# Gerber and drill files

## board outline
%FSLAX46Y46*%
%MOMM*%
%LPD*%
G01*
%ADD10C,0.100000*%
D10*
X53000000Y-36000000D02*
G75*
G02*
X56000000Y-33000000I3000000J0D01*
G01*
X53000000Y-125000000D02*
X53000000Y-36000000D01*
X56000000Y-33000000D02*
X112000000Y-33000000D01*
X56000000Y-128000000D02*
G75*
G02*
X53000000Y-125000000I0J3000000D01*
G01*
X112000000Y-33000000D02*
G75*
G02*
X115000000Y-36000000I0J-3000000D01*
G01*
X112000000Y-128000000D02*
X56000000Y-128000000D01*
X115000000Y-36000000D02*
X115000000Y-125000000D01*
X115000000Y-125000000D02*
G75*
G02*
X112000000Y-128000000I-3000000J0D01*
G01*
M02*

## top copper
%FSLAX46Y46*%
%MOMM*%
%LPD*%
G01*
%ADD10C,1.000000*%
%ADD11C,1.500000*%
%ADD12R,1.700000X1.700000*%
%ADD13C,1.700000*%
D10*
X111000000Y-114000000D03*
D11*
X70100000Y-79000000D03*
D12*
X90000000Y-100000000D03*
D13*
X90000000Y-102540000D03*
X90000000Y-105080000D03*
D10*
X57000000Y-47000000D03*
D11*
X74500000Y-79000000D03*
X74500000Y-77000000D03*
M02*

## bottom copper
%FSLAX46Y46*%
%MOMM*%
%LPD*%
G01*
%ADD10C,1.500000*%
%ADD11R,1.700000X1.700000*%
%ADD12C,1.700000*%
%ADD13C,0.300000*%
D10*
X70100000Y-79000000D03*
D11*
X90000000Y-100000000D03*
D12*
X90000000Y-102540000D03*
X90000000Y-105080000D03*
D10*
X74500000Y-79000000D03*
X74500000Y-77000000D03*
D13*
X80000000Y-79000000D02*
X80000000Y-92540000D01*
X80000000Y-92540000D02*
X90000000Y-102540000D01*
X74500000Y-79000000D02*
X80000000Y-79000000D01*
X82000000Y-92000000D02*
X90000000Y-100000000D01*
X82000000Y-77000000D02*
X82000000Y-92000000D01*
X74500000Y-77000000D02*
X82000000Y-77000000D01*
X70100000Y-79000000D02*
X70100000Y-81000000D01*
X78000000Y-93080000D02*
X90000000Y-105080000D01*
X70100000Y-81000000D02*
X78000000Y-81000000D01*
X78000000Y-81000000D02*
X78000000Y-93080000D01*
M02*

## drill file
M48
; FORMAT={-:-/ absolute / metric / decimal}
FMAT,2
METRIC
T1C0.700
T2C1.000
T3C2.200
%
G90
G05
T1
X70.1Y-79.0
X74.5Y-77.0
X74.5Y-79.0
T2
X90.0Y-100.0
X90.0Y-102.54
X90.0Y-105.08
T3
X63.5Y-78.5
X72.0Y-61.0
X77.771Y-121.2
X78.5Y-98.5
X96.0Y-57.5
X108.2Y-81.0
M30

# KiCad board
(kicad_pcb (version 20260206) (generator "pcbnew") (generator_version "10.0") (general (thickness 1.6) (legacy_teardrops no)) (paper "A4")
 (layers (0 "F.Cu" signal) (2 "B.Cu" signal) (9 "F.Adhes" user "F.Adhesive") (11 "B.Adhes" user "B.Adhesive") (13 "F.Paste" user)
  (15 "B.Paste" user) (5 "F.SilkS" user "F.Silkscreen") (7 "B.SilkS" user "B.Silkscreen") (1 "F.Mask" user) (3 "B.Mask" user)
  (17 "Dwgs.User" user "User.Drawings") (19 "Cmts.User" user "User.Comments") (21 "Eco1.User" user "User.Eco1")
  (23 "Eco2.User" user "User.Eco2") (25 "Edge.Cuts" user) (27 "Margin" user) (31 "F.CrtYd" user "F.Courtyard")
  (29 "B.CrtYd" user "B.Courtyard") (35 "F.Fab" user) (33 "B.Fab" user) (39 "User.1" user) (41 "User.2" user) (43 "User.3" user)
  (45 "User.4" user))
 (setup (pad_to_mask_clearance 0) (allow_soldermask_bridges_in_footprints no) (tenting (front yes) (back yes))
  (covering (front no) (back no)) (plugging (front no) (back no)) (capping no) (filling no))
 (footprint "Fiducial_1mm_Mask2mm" (layer "F.Cu") (at 111 114)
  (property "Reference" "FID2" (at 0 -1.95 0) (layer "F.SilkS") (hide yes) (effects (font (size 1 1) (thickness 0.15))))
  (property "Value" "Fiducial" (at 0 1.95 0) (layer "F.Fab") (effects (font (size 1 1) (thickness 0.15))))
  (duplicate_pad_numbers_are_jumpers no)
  (pad "" smd circle (at 0 0) (size 1 1) (layers "F.Cu" "F.Mask") (solder_mask_margin 0.5) (clearance 0.6)))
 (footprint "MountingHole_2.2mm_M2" (layer "F.Cu") (at 77.771 121.2)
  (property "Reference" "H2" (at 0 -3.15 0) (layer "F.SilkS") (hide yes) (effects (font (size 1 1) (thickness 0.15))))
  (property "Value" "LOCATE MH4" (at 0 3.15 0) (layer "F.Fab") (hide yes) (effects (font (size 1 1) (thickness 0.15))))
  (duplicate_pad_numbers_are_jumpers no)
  (pad "" np_thru_hole circle (at 0 0) (size 2.2 2.2) (drill 2.2) (layers "*.Cu" "*.Mask")))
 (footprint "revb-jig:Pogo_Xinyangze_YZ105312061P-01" (layer "F.Cu") (at 70.1 79)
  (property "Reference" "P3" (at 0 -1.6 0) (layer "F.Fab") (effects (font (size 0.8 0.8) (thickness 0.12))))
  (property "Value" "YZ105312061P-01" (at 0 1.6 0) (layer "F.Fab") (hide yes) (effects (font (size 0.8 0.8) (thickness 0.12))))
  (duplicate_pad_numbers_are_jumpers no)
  (pad "1" thru_hole circle (at 0 0) (size 1.5 1.5) (drill 0.7) (layers "*.Cu" "*.Mask" "F.Paste") (remove_unused_layers no) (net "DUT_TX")))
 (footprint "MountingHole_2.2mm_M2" (layer "F.Cu") (at 108.2 81)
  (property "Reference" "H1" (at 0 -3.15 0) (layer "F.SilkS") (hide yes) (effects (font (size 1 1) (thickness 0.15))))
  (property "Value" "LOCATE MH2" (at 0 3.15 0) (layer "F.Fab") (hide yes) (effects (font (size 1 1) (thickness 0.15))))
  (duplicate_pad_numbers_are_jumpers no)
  (pad "" np_thru_hole circle (at 0 0) (size 2.2 2.2) (drill 2.2) (layers "*.Cu" "*.Mask")))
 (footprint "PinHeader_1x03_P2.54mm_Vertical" (layer "F.Cu") (at 90 100)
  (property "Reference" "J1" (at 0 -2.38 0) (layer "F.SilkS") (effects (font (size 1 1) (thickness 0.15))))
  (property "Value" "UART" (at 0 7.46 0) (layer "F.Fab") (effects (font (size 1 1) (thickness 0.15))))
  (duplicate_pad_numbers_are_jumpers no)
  (pad "1" thru_hole rect (at 0 0) (size 1.7 1.7) (drill 1) (layers "*.Cu" "*.Mask") (remove_unused_layers no) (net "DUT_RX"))
  (pad "2" thru_hole circle (at 0 2.54) (size 1.7 1.7) (drill 1) (layers "*.Cu" "*.Mask") (remove_unused_layers no) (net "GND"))
  (pad "3" thru_hole circle (at 0 5.08) (size 1.7 1.7) (drill 1) (layers "*.Cu" "*.Mask") (remove_unused_layers no) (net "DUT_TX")))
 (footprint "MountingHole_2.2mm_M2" (layer "F.Cu") (at 96 57.5)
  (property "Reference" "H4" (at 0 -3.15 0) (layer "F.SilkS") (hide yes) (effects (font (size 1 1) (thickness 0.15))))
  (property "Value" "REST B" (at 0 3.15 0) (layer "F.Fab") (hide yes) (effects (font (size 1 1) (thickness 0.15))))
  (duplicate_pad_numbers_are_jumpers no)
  (pad "" np_thru_hole circle (at 0 0) (size 2.2 2.2) (drill 2.2) (layers "*.Cu" "*.Mask")))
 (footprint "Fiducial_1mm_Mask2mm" (layer "F.Cu") (at 57 47)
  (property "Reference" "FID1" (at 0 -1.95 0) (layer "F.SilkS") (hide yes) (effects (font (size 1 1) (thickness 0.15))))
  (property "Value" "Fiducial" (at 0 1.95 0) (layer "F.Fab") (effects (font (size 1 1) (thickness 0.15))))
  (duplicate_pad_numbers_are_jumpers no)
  (pad "" smd circle (at 0 0) (size 1 1) (layers "F.Cu" "F.Mask") (solder_mask_margin 0.5) (clearance 0.6)))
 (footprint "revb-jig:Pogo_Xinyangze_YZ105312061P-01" (layer "F.Cu") (at 74.5 79)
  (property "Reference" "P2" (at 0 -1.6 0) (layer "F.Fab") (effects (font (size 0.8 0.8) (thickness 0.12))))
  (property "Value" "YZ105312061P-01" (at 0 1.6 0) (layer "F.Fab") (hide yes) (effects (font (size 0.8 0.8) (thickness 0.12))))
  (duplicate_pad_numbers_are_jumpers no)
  (pad "1" thru_hole circle (at 0 0) (size 1.5 1.5) (drill 0.7) (layers "*.Cu" "*.Mask" "F.Paste") (remove_unused_layers no) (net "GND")))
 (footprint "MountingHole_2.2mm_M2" (layer "F.Cu") (at 78.5 98.5)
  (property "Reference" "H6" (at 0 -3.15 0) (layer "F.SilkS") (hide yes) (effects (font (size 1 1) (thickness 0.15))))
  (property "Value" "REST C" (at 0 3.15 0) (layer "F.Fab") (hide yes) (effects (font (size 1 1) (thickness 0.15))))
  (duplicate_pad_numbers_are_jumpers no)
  (pad "" np_thru_hole circle (at 0 0) (size 2.2 2.2) (drill 2.2) (layers "*.Cu" "*.Mask")))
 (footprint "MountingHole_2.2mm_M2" (layer "F.Cu") (at 72 61)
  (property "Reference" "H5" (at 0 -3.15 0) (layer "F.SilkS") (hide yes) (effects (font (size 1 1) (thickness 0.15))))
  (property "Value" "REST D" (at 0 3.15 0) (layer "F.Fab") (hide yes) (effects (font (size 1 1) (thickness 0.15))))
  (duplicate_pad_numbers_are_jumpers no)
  (pad "" np_thru_hole circle (at 0 0) (size 2.2 2.2) (drill 2.2) (layers "*.Cu" "*.Mask")))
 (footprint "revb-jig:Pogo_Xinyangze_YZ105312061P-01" (layer "F.Cu") (at 74.5 77)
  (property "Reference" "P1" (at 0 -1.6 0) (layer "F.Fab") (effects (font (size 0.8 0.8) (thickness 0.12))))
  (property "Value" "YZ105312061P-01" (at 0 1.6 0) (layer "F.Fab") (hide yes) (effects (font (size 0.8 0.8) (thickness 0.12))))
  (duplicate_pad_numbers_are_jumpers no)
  (pad "1" thru_hole circle (at 0 0) (size 1.5 1.5) (drill 0.7) (layers "*.Cu" "*.Mask" "F.Paste") (remove_unused_layers no) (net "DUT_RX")))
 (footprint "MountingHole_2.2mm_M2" (layer "F.Cu") (at 63.5 78.5)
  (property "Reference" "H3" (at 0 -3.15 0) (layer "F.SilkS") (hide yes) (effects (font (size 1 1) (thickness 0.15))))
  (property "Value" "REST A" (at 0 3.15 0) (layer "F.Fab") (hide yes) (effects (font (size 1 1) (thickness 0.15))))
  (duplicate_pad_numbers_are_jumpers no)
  (pad "" np_thru_hole circle (at 0 0) (size 2.2 2.2) (drill 2.2) (layers "*.Cu" "*.Mask")))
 (gr_arc (start 53 36) (mid 53.878679 33.878679) (end 56 33) (stroke (width 0.1) (type default)) (layer "Edge.Cuts"))
 (gr_line (start 53 125) (end 53 36) (stroke (width 0.1) (type default)) (layer "Edge.Cuts"))
 (gr_line (start 56 33) (end 112 33) (stroke (width 0.1) (type default)) (layer "Edge.Cuts"))
 (gr_arc (start 56 128) (mid 53.878679 127.12132) (end 53 125) (stroke (width 0.1) (type default)) (layer "Edge.Cuts"))
 (gr_arc (start 112 33) (mid 114.12132 33.878679) (end 115 36) (stroke (width 0.1) (type default)) (layer "Edge.Cuts"))
 (gr_line (start 112 128) (end 56 128) (stroke (width 0.1) (type default)) (layer "Edge.Cuts"))
 (gr_line (start 115 36) (end 115 125) (stroke (width 0.1) (type default)) (layer "Edge.Cuts"))
 (gr_arc (start 115 125) (mid 114.12132 127.12132) (end 112 128) (stroke (width 0.1) (type default)) (layer "Edge.Cuts"))
 (segment (start 80 79) (end 80 92.54) (width 0.3) (layer "B.Cu") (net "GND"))
 (segment (start 80 92.54) (end 90 102.54) (width 0.3) (layer "B.Cu") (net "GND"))
 (segment (start 74.5 79) (end 80 79) (width 0.3) (layer "B.Cu") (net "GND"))
 (segment (start 82 92) (end 90 100) (width 0.3) (layer "B.Cu") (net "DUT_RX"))
 (segment (start 82 77) (end 82 92) (width 0.3) (layer "B.Cu") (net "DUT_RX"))
 (segment (start 74.5 77) (end 82 77) (width 0.3) (layer "B.Cu") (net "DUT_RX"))
 (segment (start 70.1 79) (end 70.1 81) (width 0.3) (layer "B.Cu") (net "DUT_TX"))
 (segment (start 78 93.08) (end 90 105.08) (width 0.3) (layer "B.Cu") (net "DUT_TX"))
 (segment (start 70.1 81) (end 78 81) (width 0.3) (layer "B.Cu") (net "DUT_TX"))
 (segment (start 78 81) (end 78 93.08) (width 0.3) (layer "B.Cu") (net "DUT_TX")))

